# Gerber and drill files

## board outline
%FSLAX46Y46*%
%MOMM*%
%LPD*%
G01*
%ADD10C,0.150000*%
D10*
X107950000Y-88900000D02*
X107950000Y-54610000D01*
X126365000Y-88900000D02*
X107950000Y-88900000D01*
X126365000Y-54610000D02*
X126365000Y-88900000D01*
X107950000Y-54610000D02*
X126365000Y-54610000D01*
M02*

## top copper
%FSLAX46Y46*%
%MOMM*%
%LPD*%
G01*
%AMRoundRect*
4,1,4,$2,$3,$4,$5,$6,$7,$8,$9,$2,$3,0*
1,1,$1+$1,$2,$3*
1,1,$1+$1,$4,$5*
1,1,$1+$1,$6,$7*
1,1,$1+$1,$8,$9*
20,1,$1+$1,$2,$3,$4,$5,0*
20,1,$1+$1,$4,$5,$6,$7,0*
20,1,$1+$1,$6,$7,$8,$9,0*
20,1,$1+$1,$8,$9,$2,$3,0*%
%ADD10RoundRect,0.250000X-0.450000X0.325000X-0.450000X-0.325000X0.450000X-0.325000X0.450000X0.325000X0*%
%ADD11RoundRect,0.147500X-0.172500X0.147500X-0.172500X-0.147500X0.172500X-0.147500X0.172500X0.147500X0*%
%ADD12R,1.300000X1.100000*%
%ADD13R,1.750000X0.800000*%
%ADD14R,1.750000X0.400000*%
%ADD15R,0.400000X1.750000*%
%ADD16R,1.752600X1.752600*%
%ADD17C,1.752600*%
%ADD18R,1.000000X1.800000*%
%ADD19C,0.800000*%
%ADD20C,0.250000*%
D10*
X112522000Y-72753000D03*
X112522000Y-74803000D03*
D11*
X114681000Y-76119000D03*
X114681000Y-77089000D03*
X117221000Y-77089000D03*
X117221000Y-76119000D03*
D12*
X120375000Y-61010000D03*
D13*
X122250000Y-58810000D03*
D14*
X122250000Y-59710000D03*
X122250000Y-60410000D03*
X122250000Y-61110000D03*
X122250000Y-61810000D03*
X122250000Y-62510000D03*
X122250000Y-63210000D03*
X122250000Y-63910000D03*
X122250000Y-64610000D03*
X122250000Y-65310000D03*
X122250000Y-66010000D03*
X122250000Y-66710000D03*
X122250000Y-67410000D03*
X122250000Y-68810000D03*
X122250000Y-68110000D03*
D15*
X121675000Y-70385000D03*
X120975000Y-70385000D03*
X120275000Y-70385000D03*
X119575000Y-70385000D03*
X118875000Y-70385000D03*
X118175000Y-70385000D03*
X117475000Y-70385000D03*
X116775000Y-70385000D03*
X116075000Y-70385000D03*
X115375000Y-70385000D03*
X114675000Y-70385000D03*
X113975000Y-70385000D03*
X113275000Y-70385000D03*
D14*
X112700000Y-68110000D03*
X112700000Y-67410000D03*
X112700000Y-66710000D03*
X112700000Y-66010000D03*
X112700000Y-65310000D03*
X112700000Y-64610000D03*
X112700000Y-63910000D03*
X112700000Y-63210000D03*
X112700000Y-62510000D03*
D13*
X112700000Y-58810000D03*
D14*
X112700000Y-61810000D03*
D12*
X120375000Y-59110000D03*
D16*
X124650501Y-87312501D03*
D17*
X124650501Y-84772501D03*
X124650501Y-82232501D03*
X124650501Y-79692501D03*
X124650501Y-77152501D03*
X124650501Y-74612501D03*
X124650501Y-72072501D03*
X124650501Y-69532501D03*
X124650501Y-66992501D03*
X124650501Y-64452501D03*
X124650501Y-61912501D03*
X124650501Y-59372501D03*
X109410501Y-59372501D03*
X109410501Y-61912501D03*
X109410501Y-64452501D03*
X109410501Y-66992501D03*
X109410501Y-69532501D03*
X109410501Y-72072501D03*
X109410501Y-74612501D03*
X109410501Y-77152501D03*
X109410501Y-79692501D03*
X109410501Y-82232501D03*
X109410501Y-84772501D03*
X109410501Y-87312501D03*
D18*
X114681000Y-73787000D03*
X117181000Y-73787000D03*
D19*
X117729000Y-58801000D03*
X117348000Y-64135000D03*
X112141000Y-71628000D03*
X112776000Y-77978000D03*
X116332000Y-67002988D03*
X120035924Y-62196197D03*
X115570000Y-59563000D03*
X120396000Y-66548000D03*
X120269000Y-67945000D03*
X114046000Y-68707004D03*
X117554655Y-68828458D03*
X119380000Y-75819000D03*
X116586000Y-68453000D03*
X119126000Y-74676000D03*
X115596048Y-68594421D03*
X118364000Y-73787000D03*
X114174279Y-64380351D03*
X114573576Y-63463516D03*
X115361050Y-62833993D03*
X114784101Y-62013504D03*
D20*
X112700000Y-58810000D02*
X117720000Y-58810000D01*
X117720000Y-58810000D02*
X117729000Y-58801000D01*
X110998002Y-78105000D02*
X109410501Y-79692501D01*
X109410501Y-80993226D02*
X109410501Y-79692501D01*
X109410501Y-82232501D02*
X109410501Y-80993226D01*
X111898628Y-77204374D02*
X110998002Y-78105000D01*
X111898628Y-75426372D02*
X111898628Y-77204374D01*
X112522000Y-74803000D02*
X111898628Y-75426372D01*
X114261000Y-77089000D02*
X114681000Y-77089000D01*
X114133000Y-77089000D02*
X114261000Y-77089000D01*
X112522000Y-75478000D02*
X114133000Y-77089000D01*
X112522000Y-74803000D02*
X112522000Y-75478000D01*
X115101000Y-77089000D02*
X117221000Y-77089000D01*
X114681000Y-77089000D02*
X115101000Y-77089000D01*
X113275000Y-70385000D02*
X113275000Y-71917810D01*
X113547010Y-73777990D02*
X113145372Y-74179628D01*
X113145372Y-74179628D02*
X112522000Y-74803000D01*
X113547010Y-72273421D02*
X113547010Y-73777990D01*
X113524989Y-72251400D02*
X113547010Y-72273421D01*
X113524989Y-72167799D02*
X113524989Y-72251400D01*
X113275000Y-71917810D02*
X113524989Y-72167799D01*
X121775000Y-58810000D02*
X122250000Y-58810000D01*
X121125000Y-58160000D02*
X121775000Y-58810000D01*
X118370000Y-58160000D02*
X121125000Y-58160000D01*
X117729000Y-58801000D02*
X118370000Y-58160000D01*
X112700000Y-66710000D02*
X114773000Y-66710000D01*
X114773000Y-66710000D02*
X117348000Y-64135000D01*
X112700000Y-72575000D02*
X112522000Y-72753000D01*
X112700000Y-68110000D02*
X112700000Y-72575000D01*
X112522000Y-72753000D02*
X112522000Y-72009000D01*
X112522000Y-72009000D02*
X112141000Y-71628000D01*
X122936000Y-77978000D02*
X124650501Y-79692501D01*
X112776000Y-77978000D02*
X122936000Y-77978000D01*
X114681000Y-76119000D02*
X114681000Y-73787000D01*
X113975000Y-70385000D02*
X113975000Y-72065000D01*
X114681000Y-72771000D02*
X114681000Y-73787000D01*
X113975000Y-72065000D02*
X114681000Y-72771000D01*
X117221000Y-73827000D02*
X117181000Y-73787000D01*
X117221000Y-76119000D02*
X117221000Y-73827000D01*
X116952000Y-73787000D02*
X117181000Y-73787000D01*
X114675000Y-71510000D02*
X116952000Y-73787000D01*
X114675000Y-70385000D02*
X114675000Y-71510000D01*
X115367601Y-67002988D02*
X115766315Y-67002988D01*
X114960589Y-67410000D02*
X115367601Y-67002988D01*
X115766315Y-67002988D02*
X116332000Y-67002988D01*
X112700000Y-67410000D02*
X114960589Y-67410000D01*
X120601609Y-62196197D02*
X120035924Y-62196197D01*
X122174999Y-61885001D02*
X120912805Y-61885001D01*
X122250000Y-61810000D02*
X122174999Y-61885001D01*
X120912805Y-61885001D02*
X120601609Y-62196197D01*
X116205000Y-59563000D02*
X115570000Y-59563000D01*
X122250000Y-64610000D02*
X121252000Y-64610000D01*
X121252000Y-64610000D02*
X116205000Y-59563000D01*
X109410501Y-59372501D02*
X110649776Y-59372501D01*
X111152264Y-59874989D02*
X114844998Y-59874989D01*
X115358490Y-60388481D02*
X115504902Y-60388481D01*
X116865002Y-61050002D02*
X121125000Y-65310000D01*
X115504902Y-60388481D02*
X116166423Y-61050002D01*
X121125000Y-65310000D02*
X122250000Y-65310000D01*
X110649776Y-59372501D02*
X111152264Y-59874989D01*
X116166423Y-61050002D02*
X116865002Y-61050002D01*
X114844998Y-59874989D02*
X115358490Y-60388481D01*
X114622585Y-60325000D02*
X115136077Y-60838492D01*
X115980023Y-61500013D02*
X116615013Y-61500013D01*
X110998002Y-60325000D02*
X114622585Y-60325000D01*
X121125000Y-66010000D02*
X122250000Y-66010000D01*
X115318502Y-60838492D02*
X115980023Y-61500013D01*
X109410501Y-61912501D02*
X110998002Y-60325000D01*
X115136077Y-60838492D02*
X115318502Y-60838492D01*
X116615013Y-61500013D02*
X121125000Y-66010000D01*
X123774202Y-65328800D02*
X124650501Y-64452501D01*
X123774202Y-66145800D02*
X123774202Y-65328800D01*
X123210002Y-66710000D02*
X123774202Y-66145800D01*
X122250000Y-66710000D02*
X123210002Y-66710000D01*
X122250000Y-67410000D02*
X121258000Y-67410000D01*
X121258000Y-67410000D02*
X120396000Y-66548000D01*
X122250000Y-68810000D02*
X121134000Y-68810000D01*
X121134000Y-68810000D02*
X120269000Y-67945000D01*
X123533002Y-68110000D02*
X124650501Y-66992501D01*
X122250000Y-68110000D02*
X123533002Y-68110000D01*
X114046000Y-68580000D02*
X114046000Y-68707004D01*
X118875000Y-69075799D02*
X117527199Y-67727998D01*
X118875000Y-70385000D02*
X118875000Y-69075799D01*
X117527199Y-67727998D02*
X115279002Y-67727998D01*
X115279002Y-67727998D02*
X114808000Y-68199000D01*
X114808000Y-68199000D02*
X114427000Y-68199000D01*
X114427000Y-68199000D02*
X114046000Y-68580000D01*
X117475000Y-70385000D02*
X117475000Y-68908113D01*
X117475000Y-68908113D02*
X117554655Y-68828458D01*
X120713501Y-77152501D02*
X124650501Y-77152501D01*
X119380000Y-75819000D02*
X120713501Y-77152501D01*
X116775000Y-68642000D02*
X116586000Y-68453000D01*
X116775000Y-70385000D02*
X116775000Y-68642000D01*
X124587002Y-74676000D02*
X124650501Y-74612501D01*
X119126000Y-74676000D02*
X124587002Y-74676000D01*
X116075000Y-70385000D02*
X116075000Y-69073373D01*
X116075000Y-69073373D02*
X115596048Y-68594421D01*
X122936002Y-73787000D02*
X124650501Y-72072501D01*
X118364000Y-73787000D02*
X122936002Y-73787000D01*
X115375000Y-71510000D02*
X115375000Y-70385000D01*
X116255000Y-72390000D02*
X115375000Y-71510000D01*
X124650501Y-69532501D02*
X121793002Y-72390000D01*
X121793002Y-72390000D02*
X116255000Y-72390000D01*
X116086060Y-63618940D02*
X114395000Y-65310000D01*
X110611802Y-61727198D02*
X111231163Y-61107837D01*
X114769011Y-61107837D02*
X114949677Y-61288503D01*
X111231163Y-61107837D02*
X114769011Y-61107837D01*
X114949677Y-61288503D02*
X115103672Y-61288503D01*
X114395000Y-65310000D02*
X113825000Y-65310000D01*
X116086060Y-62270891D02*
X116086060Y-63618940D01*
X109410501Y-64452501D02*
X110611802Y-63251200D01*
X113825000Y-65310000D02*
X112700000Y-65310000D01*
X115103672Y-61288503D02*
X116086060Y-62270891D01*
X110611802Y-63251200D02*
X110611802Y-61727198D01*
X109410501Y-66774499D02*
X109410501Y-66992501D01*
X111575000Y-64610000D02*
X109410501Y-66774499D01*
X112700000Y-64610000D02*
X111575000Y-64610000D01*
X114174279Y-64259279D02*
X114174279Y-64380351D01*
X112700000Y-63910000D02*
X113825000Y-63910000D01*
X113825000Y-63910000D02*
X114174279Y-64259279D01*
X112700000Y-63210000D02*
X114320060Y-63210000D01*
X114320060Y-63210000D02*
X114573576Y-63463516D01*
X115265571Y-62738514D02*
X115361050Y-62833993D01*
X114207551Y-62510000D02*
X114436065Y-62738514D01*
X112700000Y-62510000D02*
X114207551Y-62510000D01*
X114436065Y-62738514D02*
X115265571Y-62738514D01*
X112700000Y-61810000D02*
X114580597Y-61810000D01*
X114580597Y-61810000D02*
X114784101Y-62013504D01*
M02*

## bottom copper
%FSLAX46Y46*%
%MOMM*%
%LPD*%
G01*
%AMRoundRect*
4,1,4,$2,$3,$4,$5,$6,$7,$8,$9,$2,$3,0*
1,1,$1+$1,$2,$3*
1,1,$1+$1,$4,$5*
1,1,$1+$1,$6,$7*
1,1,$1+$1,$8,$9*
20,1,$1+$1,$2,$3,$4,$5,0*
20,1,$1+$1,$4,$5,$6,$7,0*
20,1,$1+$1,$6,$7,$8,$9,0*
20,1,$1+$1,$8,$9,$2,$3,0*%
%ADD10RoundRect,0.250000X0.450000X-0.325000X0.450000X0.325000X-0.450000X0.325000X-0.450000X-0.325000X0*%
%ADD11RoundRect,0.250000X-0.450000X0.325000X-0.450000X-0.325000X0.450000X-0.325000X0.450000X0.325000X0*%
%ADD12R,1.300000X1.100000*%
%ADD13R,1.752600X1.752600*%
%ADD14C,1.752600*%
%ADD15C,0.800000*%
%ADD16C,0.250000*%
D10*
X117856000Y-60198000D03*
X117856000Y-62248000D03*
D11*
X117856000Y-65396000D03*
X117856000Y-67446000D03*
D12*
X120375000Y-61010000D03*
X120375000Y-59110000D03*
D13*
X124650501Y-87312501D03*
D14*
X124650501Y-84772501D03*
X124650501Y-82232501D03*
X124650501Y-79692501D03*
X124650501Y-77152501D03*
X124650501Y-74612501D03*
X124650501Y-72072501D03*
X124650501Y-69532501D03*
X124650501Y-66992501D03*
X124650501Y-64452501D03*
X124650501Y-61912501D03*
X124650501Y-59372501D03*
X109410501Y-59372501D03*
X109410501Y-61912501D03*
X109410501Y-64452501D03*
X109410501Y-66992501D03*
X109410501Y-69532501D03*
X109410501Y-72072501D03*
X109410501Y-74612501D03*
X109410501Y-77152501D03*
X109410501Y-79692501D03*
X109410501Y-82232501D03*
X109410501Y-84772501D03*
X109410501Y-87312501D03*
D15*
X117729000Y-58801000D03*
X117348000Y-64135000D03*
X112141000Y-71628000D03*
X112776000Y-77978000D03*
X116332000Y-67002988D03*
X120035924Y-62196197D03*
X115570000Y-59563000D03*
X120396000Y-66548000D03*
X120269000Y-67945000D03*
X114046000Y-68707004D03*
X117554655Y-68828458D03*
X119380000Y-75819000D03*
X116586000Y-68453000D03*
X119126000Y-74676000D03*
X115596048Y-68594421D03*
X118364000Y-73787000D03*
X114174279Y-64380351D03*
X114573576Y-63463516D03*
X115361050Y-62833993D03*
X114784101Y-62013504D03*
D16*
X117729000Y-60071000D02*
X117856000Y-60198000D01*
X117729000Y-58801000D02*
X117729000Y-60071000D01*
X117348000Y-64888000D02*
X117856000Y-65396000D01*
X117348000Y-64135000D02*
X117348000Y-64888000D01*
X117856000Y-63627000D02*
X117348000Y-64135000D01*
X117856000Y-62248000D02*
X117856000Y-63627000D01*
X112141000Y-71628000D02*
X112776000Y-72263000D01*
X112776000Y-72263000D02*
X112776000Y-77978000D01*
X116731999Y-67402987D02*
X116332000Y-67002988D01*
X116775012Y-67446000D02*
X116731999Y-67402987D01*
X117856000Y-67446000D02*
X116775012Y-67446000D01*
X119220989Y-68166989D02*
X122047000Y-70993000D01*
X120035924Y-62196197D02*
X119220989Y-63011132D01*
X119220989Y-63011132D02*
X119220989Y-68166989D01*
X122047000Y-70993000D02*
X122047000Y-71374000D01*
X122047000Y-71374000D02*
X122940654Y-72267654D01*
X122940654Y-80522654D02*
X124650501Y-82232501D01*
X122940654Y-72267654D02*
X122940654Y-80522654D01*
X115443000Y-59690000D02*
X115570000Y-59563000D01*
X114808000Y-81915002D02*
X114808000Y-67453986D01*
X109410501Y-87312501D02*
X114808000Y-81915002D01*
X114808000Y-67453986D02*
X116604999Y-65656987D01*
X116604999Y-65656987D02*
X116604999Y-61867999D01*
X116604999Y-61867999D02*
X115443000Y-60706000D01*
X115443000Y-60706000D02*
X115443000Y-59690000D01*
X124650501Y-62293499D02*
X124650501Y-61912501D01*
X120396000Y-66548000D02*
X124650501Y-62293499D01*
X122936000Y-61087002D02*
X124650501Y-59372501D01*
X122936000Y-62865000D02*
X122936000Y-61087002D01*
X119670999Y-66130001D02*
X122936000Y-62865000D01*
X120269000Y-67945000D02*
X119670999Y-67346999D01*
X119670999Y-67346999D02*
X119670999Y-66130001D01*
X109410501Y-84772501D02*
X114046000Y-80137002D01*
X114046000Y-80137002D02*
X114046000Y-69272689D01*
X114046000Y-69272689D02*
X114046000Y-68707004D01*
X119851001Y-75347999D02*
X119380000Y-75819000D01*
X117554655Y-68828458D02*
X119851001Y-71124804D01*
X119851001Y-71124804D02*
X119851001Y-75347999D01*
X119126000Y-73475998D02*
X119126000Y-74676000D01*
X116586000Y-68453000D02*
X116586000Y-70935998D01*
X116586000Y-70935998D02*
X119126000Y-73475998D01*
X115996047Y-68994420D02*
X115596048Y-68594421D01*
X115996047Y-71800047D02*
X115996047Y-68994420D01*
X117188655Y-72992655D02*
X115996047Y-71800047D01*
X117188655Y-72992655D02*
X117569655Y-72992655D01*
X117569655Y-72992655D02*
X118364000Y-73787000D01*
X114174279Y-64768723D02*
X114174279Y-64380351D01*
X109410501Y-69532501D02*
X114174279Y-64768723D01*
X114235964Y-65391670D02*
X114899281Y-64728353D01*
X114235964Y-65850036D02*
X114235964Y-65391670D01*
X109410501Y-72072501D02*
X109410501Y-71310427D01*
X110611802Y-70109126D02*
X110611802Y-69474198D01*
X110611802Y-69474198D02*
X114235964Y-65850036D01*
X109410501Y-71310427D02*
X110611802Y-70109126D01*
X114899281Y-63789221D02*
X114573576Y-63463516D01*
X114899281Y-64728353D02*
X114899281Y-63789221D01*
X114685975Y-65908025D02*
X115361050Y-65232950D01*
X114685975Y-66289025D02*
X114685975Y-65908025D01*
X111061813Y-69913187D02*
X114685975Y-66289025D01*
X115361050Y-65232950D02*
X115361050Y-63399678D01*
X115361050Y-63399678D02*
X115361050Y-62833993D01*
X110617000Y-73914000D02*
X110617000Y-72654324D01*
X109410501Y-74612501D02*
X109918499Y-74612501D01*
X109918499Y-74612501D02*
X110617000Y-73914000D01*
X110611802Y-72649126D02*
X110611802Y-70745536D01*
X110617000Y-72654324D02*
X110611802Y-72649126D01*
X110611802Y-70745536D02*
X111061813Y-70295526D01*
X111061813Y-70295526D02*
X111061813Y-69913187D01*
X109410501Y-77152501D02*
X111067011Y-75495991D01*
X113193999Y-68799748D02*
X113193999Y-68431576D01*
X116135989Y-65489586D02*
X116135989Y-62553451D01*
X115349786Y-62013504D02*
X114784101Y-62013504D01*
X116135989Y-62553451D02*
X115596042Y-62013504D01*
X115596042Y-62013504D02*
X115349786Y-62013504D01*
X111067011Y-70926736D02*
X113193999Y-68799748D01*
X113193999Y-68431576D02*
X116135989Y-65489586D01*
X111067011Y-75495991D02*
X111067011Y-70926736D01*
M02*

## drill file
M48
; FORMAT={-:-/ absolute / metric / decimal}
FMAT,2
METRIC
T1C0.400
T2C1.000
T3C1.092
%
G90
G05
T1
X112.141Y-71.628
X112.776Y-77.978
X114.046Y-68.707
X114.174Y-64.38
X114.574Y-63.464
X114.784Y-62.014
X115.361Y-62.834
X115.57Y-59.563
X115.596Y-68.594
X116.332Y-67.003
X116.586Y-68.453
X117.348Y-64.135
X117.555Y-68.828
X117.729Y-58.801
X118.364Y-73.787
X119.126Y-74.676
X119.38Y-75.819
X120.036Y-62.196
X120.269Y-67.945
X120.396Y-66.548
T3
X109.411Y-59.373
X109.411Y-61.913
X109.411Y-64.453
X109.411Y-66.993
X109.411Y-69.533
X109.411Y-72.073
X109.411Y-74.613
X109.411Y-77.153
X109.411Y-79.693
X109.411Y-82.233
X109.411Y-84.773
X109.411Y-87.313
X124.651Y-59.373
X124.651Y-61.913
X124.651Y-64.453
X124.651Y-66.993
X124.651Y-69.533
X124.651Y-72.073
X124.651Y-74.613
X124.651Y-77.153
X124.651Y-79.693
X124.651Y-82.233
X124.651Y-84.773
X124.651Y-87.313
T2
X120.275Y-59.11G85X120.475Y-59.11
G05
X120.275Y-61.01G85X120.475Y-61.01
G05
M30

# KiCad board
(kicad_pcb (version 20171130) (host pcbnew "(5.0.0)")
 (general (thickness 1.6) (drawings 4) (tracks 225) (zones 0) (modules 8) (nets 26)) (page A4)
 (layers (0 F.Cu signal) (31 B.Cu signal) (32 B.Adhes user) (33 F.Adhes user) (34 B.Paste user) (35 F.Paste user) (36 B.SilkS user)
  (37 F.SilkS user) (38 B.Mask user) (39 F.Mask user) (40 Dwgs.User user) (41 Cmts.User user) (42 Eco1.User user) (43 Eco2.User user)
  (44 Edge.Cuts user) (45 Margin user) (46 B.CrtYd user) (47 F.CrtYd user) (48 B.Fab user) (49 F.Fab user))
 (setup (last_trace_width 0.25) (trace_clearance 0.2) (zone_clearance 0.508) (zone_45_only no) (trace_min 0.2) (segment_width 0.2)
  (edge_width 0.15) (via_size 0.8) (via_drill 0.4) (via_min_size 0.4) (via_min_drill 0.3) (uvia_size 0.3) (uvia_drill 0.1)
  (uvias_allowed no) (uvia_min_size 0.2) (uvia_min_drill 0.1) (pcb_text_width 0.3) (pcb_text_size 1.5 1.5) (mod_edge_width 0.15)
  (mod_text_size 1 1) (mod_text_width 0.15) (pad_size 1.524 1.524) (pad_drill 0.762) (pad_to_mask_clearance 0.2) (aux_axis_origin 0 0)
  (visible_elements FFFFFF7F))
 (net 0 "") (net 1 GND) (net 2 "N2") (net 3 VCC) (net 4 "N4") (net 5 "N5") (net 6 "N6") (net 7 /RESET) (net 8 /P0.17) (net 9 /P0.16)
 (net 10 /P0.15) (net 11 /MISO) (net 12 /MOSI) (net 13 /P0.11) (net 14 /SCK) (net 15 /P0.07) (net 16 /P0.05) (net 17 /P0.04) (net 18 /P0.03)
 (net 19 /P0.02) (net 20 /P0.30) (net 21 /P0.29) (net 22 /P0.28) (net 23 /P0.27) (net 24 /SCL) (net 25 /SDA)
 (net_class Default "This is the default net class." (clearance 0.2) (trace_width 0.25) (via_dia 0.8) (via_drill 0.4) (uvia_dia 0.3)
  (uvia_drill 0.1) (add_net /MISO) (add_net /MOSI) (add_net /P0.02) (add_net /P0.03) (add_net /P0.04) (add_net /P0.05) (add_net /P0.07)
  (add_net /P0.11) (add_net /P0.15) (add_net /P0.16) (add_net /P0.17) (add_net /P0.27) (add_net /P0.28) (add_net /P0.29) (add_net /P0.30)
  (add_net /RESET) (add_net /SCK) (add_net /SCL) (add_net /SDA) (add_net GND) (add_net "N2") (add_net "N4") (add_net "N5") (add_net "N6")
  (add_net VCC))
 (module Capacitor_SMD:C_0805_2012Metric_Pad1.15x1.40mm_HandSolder (layer B.Cu) (at 117.856 61.223 90)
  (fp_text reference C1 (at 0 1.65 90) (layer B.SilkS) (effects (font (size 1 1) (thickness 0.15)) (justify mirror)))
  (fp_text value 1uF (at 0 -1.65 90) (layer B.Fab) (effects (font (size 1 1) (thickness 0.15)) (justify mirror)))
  (pad 2 smd roundrect (at 1.025 0 90) (size 1.15 1.4) (layers B.Cu B.Paste B.Mask) (roundrect_rratio 0.217391) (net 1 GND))
  (pad 1 smd roundrect (at -1.025 0 90) (size 1.15 1.4) (layers B.Cu B.Paste B.Mask) (roundrect_rratio 0.217391) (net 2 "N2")))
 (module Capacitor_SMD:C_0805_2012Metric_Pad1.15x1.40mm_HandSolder (layer F.Cu) (at 112.522 73.778 270)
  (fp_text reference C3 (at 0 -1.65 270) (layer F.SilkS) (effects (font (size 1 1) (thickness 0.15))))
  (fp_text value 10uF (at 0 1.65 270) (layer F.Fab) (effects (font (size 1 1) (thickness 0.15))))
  (pad 1 smd roundrect (at -1.025 0 270) (size 1.15 1.4) (layers F.Cu F.Paste F.Mask) (roundrect_rratio 0.217391) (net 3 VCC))
  (pad 2 smd roundrect (at 1.025 0 270) (size 1.15 1.4) (layers F.Cu F.Paste F.Mask) (roundrect_rratio 0.217391) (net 1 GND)))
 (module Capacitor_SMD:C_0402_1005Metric (layer F.Cu) (at 114.681 76.604 270)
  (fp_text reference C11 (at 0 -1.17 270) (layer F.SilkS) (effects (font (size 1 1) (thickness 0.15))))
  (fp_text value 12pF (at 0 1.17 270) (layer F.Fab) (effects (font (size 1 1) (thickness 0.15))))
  (pad 1 smd roundrect (at -0.485 0 270) (size 0.59 0.64) (layers F.Cu F.Paste F.Mask) (roundrect_rratio 0.25) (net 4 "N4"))
  (pad 2 smd roundrect (at 0.485 0 270) (size 0.59 0.64) (layers F.Cu F.Paste F.Mask) (roundrect_rratio 0.25) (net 1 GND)))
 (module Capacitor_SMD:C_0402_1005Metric (layer F.Cu) (at 117.221 76.604 270)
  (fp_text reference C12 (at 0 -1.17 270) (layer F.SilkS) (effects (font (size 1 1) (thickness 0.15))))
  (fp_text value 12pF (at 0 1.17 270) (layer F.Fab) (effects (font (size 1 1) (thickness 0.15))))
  (pad 2 smd roundrect (at 0.485 0 270) (size 0.59 0.64) (layers F.Cu F.Paste F.Mask) (roundrect_rratio 0.25) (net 1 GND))
  (pad 1 smd roundrect (at -0.485 0 270) (size 0.59 0.64) (layers F.Cu F.Paste F.Mask) (roundrect_rratio 0.25) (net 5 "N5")))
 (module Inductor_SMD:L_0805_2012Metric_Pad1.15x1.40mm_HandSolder (layer B.Cu) (at 117.856 66.421 270)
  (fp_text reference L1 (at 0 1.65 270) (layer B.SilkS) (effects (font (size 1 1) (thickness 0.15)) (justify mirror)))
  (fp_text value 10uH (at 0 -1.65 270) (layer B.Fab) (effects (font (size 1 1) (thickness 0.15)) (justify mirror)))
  (pad 1 smd roundrect (at -1.025 0 270) (size 1.15 1.4) (layers B.Cu B.Paste B.Mask) (roundrect_rratio 0.217391) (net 2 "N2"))
  (pad 2 smd roundrect (at 1.025 0 270) (size 1.15 1.4) (layers B.Cu B.Paste B.Mask) (roundrect_rratio 0.217391) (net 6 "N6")))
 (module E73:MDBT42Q (layer F.Cu) (at 117.475 54.61)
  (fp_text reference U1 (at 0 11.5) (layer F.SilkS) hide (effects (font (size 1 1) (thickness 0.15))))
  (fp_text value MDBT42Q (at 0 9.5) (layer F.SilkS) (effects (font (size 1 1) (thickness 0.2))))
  (pad 41 thru_hole rect (at 2.9 6.4) (size 1.3 1.1) (drill oval 1.2 1) (layers *.Cu *.Mask))
  (pad 39 smd rect (at 4.775 4.2) (size 1.75 0.8) (layers F.Cu F.Paste F.Mask) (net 1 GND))
  (pad 38 smd rect (at 4.775 5.1) (size 1.75 0.4) (layers F.Cu F.Paste F.Mask))
  (pad 37 smd rect (at 4.775 5.8) (size 1.75 0.4) (layers F.Cu F.Paste F.Mask))
  (pad 36 smd rect (at 4.775 6.5) (size 1.75 0.4) (layers F.Cu F.Paste F.Mask))
  (pad 35 smd rect (at 4.775 7.2) (size 1.75 0.4) (layers F.Cu F.Paste F.Mask) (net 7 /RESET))
  (pad 34 smd rect (at 4.775 7.9) (size 1.75 0.4) (layers F.Cu F.Paste F.Mask))
  (pad 33 smd rect (at 4.775 8.6) (size 1.75 0.4) (layers F.Cu F.Paste F.Mask))
  (pad 32 smd rect (at 4.775 9.3) (size 1.75 0.4) (layers F.Cu F.Paste F.Mask))
  (pad 31 smd rect (at 4.775 10) (size 1.75 0.4) (layers F.Cu F.Paste F.Mask) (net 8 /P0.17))
  (pad 30 smd rect (at 4.775 10.7) (size 1.75 0.4) (layers F.Cu F.Paste F.Mask) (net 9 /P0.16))
  (pad 29 smd rect (at 4.775 11.4) (size 1.75 0.4) (layers F.Cu F.Paste F.Mask) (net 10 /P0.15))
  (pad 28 smd rect (at 4.775 12.1) (size 1.75 0.4) (layers F.Cu F.Paste F.Mask) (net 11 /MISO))
  (pad 27 smd rect (at 4.775 12.8) (size 1.75 0.4) (layers F.Cu F.Paste F.Mask) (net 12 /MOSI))
  (pad 25 smd rect (at 4.775 14.2) (size 1.75 0.4) (layers F.Cu F.Paste F.Mask) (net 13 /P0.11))
  (pad 26 smd rect (at 4.775 13.5) (size 1.75 0.4) (layers F.Cu F.Paste F.Mask) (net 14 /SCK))
  (pad 24 smd rect (at 4.2 15.775) (size 0.4 1.75) (layers F.Cu F.Paste F.Mask) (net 1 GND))
  (pad 23 smd rect (at 3.5 15.775) (size 0.4 1.75) (layers F.Cu F.Paste F.Mask))
  (pad 22 smd rect (at 2.8 15.775) (size 0.4 1.75) (layers F.Cu F.Paste F.Mask))
  (pad 21 smd rect (at 2.1 15.775) (size 0.4 1.75) (layers F.Cu F.Paste F.Mask))
  (pad 20 smd rect (at 1.4 15.775) (size 0.4 1.75) (layers F.Cu F.Paste F.Mask) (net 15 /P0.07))
  (pad 19 smd rect (at 0.7 15.775) (size 0.4 1.75) (layers F.Cu F.Paste F.Mask))
  (pad 18 smd rect (at 0 15.775) (size 0.4 1.75) (layers F.Cu F.Paste F.Mask) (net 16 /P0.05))
  (pad 17 smd rect (at -0.7 15.775) (size 0.4 1.75) (layers F.Cu F.Paste F.Mask) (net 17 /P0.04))
  (pad 16 smd rect (at -1.4 15.775) (size 0.4 1.75) (layers F.Cu F.Paste F.Mask) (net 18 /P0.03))
  (pad 15 smd rect (at -2.1 15.775) (size 0.4 1.75) (layers F.Cu F.Paste F.Mask) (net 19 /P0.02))
  (pad 14 smd rect (at -2.8 15.775) (size 0.4 1.75) (layers F.Cu F.Paste F.Mask) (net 5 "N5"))
  (pad 13 smd rect (at -3.5 15.775) (size 0.4 1.75) (layers F.Cu F.Paste F.Mask) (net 4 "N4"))
  (pad 12 smd rect (at -4.2 15.775) (size 0.4 1.75) (layers F.Cu F.Paste F.Mask) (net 1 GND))
  (pad 11 smd rect (at -4.775 13.5) (size 1.75 0.4) (layers F.Cu F.Paste F.Mask) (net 3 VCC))
  (pad 10 smd rect (at -4.775 12.8) (size 1.75 0.4) (layers F.Cu F.Paste F.Mask) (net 6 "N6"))
  (pad 9 smd rect (at -4.775 12.1) (size 1.75 0.4) (layers F.Cu F.Paste F.Mask) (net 2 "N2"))
  (pad 8 smd rect (at -4.775 11.4) (size 1.75 0.4) (layers F.Cu F.Paste F.Mask))
  (pad 7 smd rect (at -4.775 10.7) (size 1.75 0.4) (layers F.Cu F.Paste F.Mask) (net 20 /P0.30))
  (pad 6 smd rect (at -4.775 10) (size 1.75 0.4) (layers F.Cu F.Paste F.Mask) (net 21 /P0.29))
  (pad 5 smd rect (at -4.775 9.3) (size 1.75 0.4) (layers F.Cu F.Paste F.Mask) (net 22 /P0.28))
  (pad 4 smd rect (at -4.775 8.6) (size 1.75 0.4) (layers F.Cu F.Paste F.Mask) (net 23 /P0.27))
  (pad 3 smd rect (at -4.775 7.9) (size 1.75 0.4) (layers F.Cu F.Paste F.Mask) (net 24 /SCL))
  (pad 1 smd rect (at -4.775 4.2) (size 1.75 0.8) (layers F.Cu F.Paste F.Mask) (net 1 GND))
  (pad 2 smd rect (at -4.775 7.2) (size 1.75 0.4) (layers F.Cu F.Paste F.Mask) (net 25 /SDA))
  (pad 40 thru_hole rect (at 2.9 4.5) (size 1.3 1.1) (drill oval 1.2 1) (layers *.Cu *.Mask)))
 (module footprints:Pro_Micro (layer F.Cu) (at 117.030501 74.866501 180)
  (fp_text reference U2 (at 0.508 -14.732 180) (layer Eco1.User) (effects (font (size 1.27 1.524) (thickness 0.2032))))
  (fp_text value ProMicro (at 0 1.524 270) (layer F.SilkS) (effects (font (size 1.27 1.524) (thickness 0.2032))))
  (pad 1 thru_hole rect (at -7.62 -12.446 90) (size 1.7526 1.7526) (drill 1.0922) (layers *.Cu *.SilkS *.Mask))
  (pad 2 thru_hole circle (at -7.62 -9.906 90) (size 1.7526 1.7526) (drill 1.0922) (layers *.Cu *.SilkS *.Mask) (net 1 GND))
  (pad 3 thru_hole circle (at -7.62 -7.366 90) (size 1.7526 1.7526) (drill 1.0922) (layers *.Cu *.SilkS *.Mask) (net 7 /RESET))
  (pad 4 thru_hole circle (at -7.62 -4.826 90) (size 1.7526 1.7526) (drill 1.0922) (layers *.Cu *.SilkS *.Mask) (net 3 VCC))
  (pad 5 thru_hole circle (at -7.62 -2.286 90) (size 1.7526 1.7526) (drill 1.0922) (layers *.Cu *.SilkS *.Mask) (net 16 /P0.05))
  (pad 6 thru_hole circle (at -7.62 0.254 90) (size 1.7526 1.7526) (drill 1.0922) (layers *.Cu *.SilkS *.Mask) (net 17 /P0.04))
  (pad 7 thru_hole circle (at -7.62 2.794 90) (size 1.7526 1.7526) (drill 1.0922) (layers *.Cu *.SilkS *.Mask) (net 18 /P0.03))
  (pad 8 thru_hole circle (at -7.62 5.334 90) (size 1.7526 1.7526) (drill 1.0922) (layers *.Cu *.SilkS *.Mask) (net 19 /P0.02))
  (pad 9 thru_hole circle (at -7.62 7.874 90) (size 1.7526 1.7526) (drill 1.0922) (layers *.Cu *.SilkS *.Mask) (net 14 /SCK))
  (pad 10 thru_hole circle (at -7.62 10.414 90) (size 1.7526 1.7526) (drill 1.0922) (layers *.Cu *.SilkS *.Mask) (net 11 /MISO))
  (pad 11 thru_hole circle (at -7.62 12.954 90) (size 1.7526 1.7526) (drill 1.0922) (layers *.Cu *.SilkS *.Mask) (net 12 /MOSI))
  (pad 12 thru_hole circle (at -7.62 15.494 90) (size 1.7526 1.7526) (drill 1.0922) (layers *.Cu *.SilkS *.Mask) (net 13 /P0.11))
  (pad 24 thru_hole circle (at 7.62 15.494 90) (size 1.7526 1.7526) (drill 1.0922) (layers *.Cu *.SilkS *.Mask) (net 9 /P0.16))
  (pad 23 thru_hole circle (at 7.62 12.954 90) (size 1.7526 1.7526) (drill 1.0922) (layers *.Cu *.SilkS *.Mask) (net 10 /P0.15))
  (pad 22 thru_hole circle (at 7.62 10.414 90) (size 1.7526 1.7526) (drill 1.0922) (layers *.Cu *.SilkS *.Mask) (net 20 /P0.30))
  (pad 21 thru_hole circle (at 7.62 7.874 90) (size 1.7526 1.7526) (drill 1.0922) (layers *.Cu *.SilkS *.Mask) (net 21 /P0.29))
  (pad 20 thru_hole circle (at 7.62 5.334 90) (size 1.7526 1.7526) (drill 1.0922) (layers *.Cu *.SilkS *.Mask) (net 22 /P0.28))
  (pad 19 thru_hole circle (at 7.62 2.794 90) (size 1.7526 1.7526) (drill 1.0922) (layers *.Cu *.SilkS *.Mask) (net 23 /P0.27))
  (pad 18 thru_hole circle (at 7.62 0.254 90) (size 1.7526 1.7526) (drill 1.0922) (layers *.Cu *.SilkS *.Mask) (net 24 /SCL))
  (pad 17 thru_hole circle (at 7.62 -2.286 90) (size 1.7526 1.7526) (drill 1.0922) (layers *.Cu *.SilkS *.Mask) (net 25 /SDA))
  (pad 16 thru_hole circle (at 7.62 -4.826 90) (size 1.7526 1.7526) (drill 1.0922) (layers *.Cu *.SilkS *.Mask) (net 1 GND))
  (pad 15 thru_hole circle (at 7.62 -7.366 90) (size 1.7526 1.7526) (drill 1.0922) (layers *.Cu *.SilkS *.Mask) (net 1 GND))
  (pad 14 thru_hole circle (at 7.62 -9.906 90) (size 1.7526 1.7526) (drill 1.0922) (layers *.Cu *.SilkS *.Mask) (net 15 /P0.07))
  (pad 13 thru_hole circle (at 7.62 -12.446 90) (size 1.7526 1.7526) (drill 1.0922) (layers *.Cu *.SilkS *.Mask) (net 8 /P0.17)))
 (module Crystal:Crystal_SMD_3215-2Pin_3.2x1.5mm (layer F.Cu) (at 115.931 73.787 180)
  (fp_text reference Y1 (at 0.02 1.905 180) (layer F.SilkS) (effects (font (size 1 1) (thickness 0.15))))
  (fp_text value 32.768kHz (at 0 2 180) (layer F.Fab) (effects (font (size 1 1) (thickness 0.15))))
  (pad 1 smd rect (at 1.25 0 180) (size 1 1.8) (layers F.Cu F.Paste F.Mask) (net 4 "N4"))
  (pad 2 smd rect (at -1.25 0 180) (size 1 1.8) (layers F.Cu F.Paste F.Mask) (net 5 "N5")))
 (gr_line (start 107.95 88.9) (end 107.95 54.61) (layer Edge.Cuts) (width 0.15))
 (gr_line (start 126.365 88.9) (end 107.95 88.9) (layer Edge.Cuts) (width 0.15))
 (gr_line (start 126.365 54.61) (end 126.365 88.9) (layer Edge.Cuts) (width 0.15))
 (gr_line (start 107.95 54.61) (end 126.365 54.61) (layer Edge.Cuts) (width 0.15))
 (via (at 117.729 58.801) (size 0.8) (drill 0.4) (layers F.Cu B.Cu) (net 1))
 (segment (start 112.7 58.81) (end 117.72 58.81) (width 0.25) (layer F.Cu) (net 1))
 (segment (start 117.72 58.81) (end 117.729 58.801) (width 0.25) (layer F.Cu) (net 1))
 (segment (start 117.729 60.071) (end 117.856 60.198) (width 0.25) (layer B.Cu) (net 1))
 (segment (start 117.729 58.801) (end 117.729 60.071) (width 0.25) (layer B.Cu) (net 1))
 (segment (start 110.998002 78.105) (end 109.410501 79.692501) (width 0.25) (layer F.Cu) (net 1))
 (segment (start 109.410501 80.993226) (end 109.410501 79.692501) (width 0.25) (layer F.Cu) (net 1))
 (segment (start 109.410501 82.232501) (end 109.410501 80.993226) (width 0.25) (layer F.Cu) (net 1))
 (segment (start 111.898628 77.204374) (end 110.998002 78.105) (width 0.25) (layer F.Cu) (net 1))
 (segment (start 111.898628 75.426372) (end 111.898628 77.204374) (width 0.25) (layer F.Cu) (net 1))
 (segment (start 112.522 74.803) (end 111.898628 75.426372) (width 0.25) (layer F.Cu) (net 1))
 (segment (start 114.261 77.089) (end 114.681 77.089) (width 0.25) (layer F.Cu) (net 1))
 (segment (start 114.133 77.089) (end 114.261 77.089) (width 0.25) (layer F.Cu) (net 1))
 (segment (start 112.522 75.478) (end 114.133 77.089) (width 0.25) (layer F.Cu) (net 1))
 (segment (start 112.522 74.803) (end 112.522 75.478) (width 0.25) (layer F.Cu) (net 1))
 (segment (start 115.101 77.089) (end 117.221 77.089) (width 0.25) (layer F.Cu) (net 1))
 (segment (start 114.681 77.089) (end 115.101 77.089) (width 0.25) (layer F.Cu) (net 1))
 (segment (start 113.275 70.385) (end 113.275 71.91781) (width 0.25) (layer F.Cu) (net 1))
 (segment (start 113.54701 73.77799) (end 113.145372 74.179628) (width 0.25) (layer F.Cu) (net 1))
 (segment (start 113.145372 74.179628) (end 112.522 74.803) (width 0.25) (layer F.Cu) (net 1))
 (segment (start 113.54701 72.273421) (end 113.54701 73.77799) (width 0.25) (layer F.Cu) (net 1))
 (segment (start 113.524989 72.2514) (end 113.54701 72.273421) (width 0.25) (layer F.Cu) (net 1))
 (segment (start 113.524989 72.167799) (end 113.524989 72.2514) (width 0.25) (layer F.Cu) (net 1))
 (segment (start 113.275 71.91781) (end 113.524989 72.167799) (width 0.25) (layer F.Cu) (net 1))
 (segment (start 121.775 58.81) (end 122.25 58.81) (width 0.25) (layer F.Cu) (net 1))
 (segment (start 121.125 58.16) (end 121.775 58.81) (width 0.25) (layer F.Cu) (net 1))
 (segment (start 118.37 58.16) (end 121.125 58.16) (width 0.25) (layer F.Cu) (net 1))
 (segment (start 117.729 58.801) (end 118.37 58.16) (width 0.25) (layer F.Cu) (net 1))
 (via (at 117.348 64.135) (size 0.8) (drill 0.4) (layers F.Cu B.Cu) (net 2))
 (segment (start 112.7 66.71) (end 114.773 66.71) (width 0.25) (layer F.Cu) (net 2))
 (segment (start 114.773 66.71) (end 117.348 64.135) (width 0.25) (layer F.Cu) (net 2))
 (segment (start 117.348 64.888) (end 117.856 65.396) (width 0.25) (layer B.Cu) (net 2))
 (segment (start 117.348 64.135) (end 117.348 64.888) (width 0.25) (layer B.Cu) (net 2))
 (segment (start 117.856 63.627) (end 117.348 64.135) (width 0.25) (layer B.Cu) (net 2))
 (segment (start 117.856 62.248) (end 117.856 63.627) (width 0.25) (layer B.Cu) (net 2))
 (segment (start 112.7 72.575) (end 112.522 72.753) (width 0.25) (layer F.Cu) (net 3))
 (segment (start 112.7 68.11) (end 112.7 72.575) (width 0.25) (layer F.Cu) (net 3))
 (via (at 112.141 71.628) (size 0.8) (drill 0.4) (layers F.Cu B.Cu) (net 3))
 (segment (start 112.522 72.753) (end 112.522 72.009) (width 0.25) (layer F.Cu) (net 3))
 (segment (start 112.522 72.009) (end 112.141 71.628) (width 0.25) (layer F.Cu) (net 3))
 (via (at 112.776 77.978) (size 0.8) (drill 0.4) (layers F.Cu B.Cu) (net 3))
 (segment (start 112.141 71.628) (end 112.776 72.263) (width 0.25) (layer B.Cu) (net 3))
 (segment (start 112.776 72.263) (end 112.776 77.978) (width 0.25) (layer B.Cu) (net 3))
 (segment (start 122.936 77.978) (end 124.650501 79.692501) (width 0.25) (layer F.Cu) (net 3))
 (segment (start 112.776 77.978) (end 122.936 77.978) (width 0.25) (layer F.Cu) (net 3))
 (segment (start 114.681 76.119) (end 114.681 73.787) (width 0.25) (layer F.Cu) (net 4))
 (segment (start 113.975 70.385) (end 113.975 72.065) (width 0.25) (layer F.Cu) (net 4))
 (segment (start 114.681 72.771) (end 114.681 73.787) (width 0.25) (layer F.Cu) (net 4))
 (segment (start 113.975 72.065) (end 114.681 72.771) (width 0.25) (layer F.Cu) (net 4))
 (segment (start 117.221 73.827) (end 117.181 73.787) (width 0.25) (layer F.Cu) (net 5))
 (segment (start 117.221 76.119) (end 117.221 73.827) (width 0.25) (layer F.Cu) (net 5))
 (segment (start 116.952 73.787) (end 117.181 73.787) (width 0.25) (layer F.Cu) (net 5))
 (segment (start 114.675 71.51) (end 116.952 73.787) (width 0.25) (layer F.Cu) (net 5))
 (segment (start 114.675 70.385) (end 114.675 71.51) (width 0.25) (layer F.Cu) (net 5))
 (via (at 116.332 67.002988) (size 0.8) (drill 0.4) (layers F.Cu B.Cu) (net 6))
 (segment (start 116.731999 67.402987) (end 116.332 67.002988) (width 0.25) (layer B.Cu) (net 6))
 (segment (start 116.775012 67.446) (end 116.731999 67.402987) (width 0.25) (layer B.Cu) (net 6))
 (segment (start 117.856 67.446) (end 116.775012 67.446) (width 0.25) (layer B.Cu) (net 6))
 (segment (start 115.367601 67.002988) (end 115.766315 67.002988) (width 0.25) (layer F.Cu) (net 6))
 (segment (start 114.960589 67.41) (end 115.367601 67.002988) (width 0.25) (layer F.Cu) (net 6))
 (segment (start 115.766315 67.002988) (end 116.332 67.002988) (width 0.25) (layer F.Cu) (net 6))
 (segment (start 112.7 67.41) (end 114.960589 67.41) (width 0.25) (layer F.Cu) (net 6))
 (segment (start 120.601609 62.196197) (end 120.035924 62.196197) (width 0.25) (layer F.Cu) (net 7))
 (segment (start 122.174999 61.885001) (end 120.912805 61.885001) (width 0.25) (layer F.Cu) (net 7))
 (segment (start 122.25 61.81) (end 122.174999 61.885001) (width 0.25) (layer F.Cu) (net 7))
 (segment (start 120.912805 61.885001) (end 120.601609 62.196197) (width 0.25) (layer F.Cu) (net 7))
 (via (at 120.035924 62.196197) (size 0.8) (drill 0.4) (layers F.Cu B.Cu) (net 7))
 (segment (start 119.220989 68.166989) (end 122.047 70.993) (width 0.25) (layer B.Cu) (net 7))
 (segment (start 120.035924 62.196197) (end 119.220989 63.011132) (width 0.25) (layer B.Cu) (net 7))
 (segment (start 119.220989 63.011132) (end 119.220989 68.166989) (width 0.25) (layer B.Cu) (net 7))
 (segment (start 122.047 70.993) (end 122.047 71.374) (width 0.25) (layer B.Cu) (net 7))
 (segment (start 122.047 71.374) (end 122.940654 72.267654) (width 0.25) (layer B.Cu) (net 7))
 (segment (start 122.940654 80.522654) (end 124.650501 82.232501) (width 0.25) (layer B.Cu) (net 7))
 (segment (start 122.940654 72.267654) (end 122.940654 80.522654) (width 0.25) (layer B.Cu) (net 7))
 (via (at 115.57 59.563) (size 0.8) (drill 0.4) (layers F.Cu B.Cu) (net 8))
 (segment (start 115.443 59.69) (end 115.57 59.563) (width 0.25) (layer B.Cu) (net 8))
 (segment (start 114.808 81.915002) (end 114.808 67.453986) (width 0.25) (layer B.Cu) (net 8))
 (segment (start 109.410501 87.312501) (end 114.808 81.915002) (width 0.25) (layer B.Cu) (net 8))
 (segment (start 114.808 67.453986) (end 116.604999 65.656987) (width 0.25) (layer B.Cu) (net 8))
 (segment (start 116.604999 65.656987) (end 116.604999 61.867999) (width 0.25) (layer B.Cu) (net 8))
 (segment (start 116.604999 61.867999) (end 115.443 60.706) (width 0.25) (layer B.Cu) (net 8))
 (segment (start 115.443 60.706) (end 115.443 59.69) (width 0.25) (layer B.Cu) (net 8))
 (segment (start 116.205 59.563) (end 115.57 59.563) (width 0.25) (layer F.Cu) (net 8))
 (segment (start 122.25 64.61) (end 121.252 64.61) (width 0.25) (layer F.Cu) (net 8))
 (segment (start 121.252 64.61) (end 116.205 59.563) (width 0.25) (layer F.Cu) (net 8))
 (segment (start 109.410501 59.372501) (end 110.649776 59.372501) (width 0.25) (layer F.Cu) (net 9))
 (segment (start 111.152264 59.874989) (end 114.844998 59.874989) (width 0.25) (layer F.Cu) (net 9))
 (segment (start 115.35849 60.388481) (end 115.504902 60.388481) (width 0.25) (layer F.Cu) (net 9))
 (segment (start 116.865002 61.050002) (end 121.125 65.31) (width 0.25) (layer F.Cu) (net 9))
 (segment (start 115.504902 60.388481) (end 116.166423 61.050002) (width 0.25) (layer F.Cu) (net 9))
 (segment (start 121.125 65.31) (end 122.25 65.31) (width 0.25) (layer F.Cu) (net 9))
 (segment (start 110.649776 59.372501) (end 111.152264 59.874989) (width 0.25) (layer F.Cu) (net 9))
 (segment (start 116.166423 61.050002) (end 116.865002 61.050002) (width 0.25) (layer F.Cu) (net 9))
 (segment (start 114.844998 59.874989) (end 115.35849 60.388481) (width 0.25) (layer F.Cu) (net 9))
 (segment (start 114.622585 60.325) (end 115.136077 60.838492) (width 0.25) (layer F.Cu) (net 10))
 (segment (start 115.980023 61.500013) (end 116.615013 61.500013) (width 0.25) (layer F.Cu) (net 10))
 (segment (start 110.998002 60.325) (end 114.622585 60.325) (width 0.25) (layer F.Cu) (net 10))
 (segment (start 121.125 66.01) (end 122.25 66.01) (width 0.25) (layer F.Cu) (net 10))
 (segment (start 115.318502 60.838492) (end 115.980023 61.500013) (width 0.25) (layer F.Cu) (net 10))
 (segment (start 109.410501 61.912501) (end 110.998002 60.325) (width 0.25) (layer F.Cu) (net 10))
 (segment (start 115.136077 60.838492) (end 115.318502 60.838492) (width 0.25) (layer F.Cu) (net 10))
 (segment (start 116.615013 61.500013) (end 121.125 66.01) (width 0.25) (layer F.Cu) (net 10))
 (segment (start 123.774202 65.3288) (end 124.650501 64.452501) (width 0.25) (layer F.Cu) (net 11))
 (segment (start 123.774202 66.1458) (end 123.774202 65.3288) (width 0.25) (layer F.Cu) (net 11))
 (segment (start 123.210002 66.71) (end 123.774202 66.1458) (width 0.25) (layer F.Cu) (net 11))
 (segment (start 122.25 66.71) (end 123.210002 66.71) (width 0.25) (layer F.Cu) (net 11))
 (via (at 120.396 66.548) (size 0.8) (drill 0.4) (layers F.Cu B.Cu) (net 12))
 (segment (start 122.25 67.41) (end 121.258 67.41) (width 0.25) (layer F.Cu) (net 12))
 (segment (start 121.258 67.41) (end 120.396 66.548) (width 0.25) (layer F.Cu) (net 12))
 (segment (start 124.650501 62.293499) (end 124.650501 61.912501) (width 0.25) (layer B.Cu) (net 12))
 (segment (start 120.396 66.548) (end 124.650501 62.293499) (width 0.25) (layer B.Cu) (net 12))
 (via (at 120.269 67.945) (size 0.8) (drill 0.4) (layers F.Cu B.Cu) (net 13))
 (segment (start 122.25 68.81) (end 121.134 68.81) (width 0.25) (layer F.Cu) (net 13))
 (segment (start 121.134 68.81) (end 120.269 67.945) (width 0.25) (layer F.Cu) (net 13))
 (segment (start 122.936 61.087002) (end 124.650501 59.372501) (width 0.25) (layer B.Cu) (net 13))
 (segment (start 122.936 62.865) (end 122.936 61.087002) (width 0.25) (layer B.Cu) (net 13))
 (segment (start 119.670999 66.130001) (end 122.936 62.865) (width 0.25) (layer B.Cu) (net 13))
 (segment (start 120.269 67.945) (end 119.670999 67.346999) (width 0.25) (layer B.Cu) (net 13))
 (segment (start 119.670999 67.346999) (end 119.670999 66.130001) (width 0.25) (layer B.Cu) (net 13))
 (segment (start 123.533002 68.11) (end 124.650501 66.992501) (width 0.25) (layer F.Cu) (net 14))
 (segment (start 122.25 68.11) (end 123.533002 68.11) (width 0.25) (layer F.Cu) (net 14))
 (segment (start 109.410501 84.772501) (end 114.046 80.137002) (width 0.25) (layer B.Cu) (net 15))
 (via (at 114.046 68.707004) (size 0.8) (drill 0.4) (layers F.Cu B.Cu) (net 15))
 (segment (start 114.046 80.137002) (end 114.046 69.272689) (width 0.25) (layer B.Cu) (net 15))
 (segment (start 114.046 69.272689) (end 114.046 68.707004) (width 0.25) (layer B.Cu) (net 15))
 (segment (start 114.046 68.58) (end 114.046 68.707004) (width 0.25) (layer F.Cu) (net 15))
 (segment (start 118.875 69.075799) (end 117.527199 67.727998) (width 0.25) (layer F.Cu) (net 15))
 (segment (start 118.875 70.385) (end 118.875 69.075799) (width 0.25) (layer F.Cu) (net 15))
 (segment (start 117.527199 67.727998) (end 115.279002 67.727998) (width 0.25) (layer F.Cu) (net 15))
 (segment (start 115.279002 67.727998) (end 114.808 68.199) (width 0.25) (layer F.Cu) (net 15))
 (segment (start 114.808 68.199) (end 114.427 68.199) (width 0.25) (layer F.Cu) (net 15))
 (segment (start 114.427 68.199) (end 114.046 68.58) (width 0.25) (layer F.Cu) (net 15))
 (segment (start 117.475 70.385) (end 117.475 68.908113) (width 0.25) (layer F.Cu) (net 16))
 (segment (start 117.475 68.908113) (end 117.554655 68.828458) (width 0.25) (layer F.Cu) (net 16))
 (via (at 117.554655 68.828458) (size 0.8) (drill 0.4) (layers F.Cu B.Cu) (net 16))
 (via (at 119.38 75.819) (size 0.8) (drill 0.4) (layers F.Cu B.Cu) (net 16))
 (segment (start 119.851001 75.347999) (end 119.38 75.819) (width 0.25) (layer B.Cu) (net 16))
 (segment (start 117.554655 68.828458) (end 119.851001 71.124804) (width 0.25) (layer B.Cu) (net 16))
 (segment (start 119.851001 71.124804) (end 119.851001 75.347999) (width 0.25) (layer B.Cu) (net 16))
 (segment (start 120.713501 77.152501) (end 124.650501 77.152501) (width 0.25) (layer F.Cu) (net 16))
 (segment (start 119.38 75.819) (end 120.713501 77.152501) (width 0.25) (layer F.Cu) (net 16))
 (segment (start 116.775 68.642) (end 116.586 68.453) (width 0.25) (layer F.Cu) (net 17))
 (via (at 116.586 68.453) (size 0.8) (drill 0.4) (layers F.Cu B.Cu) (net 17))
 (segment (start 116.775 70.385) (end 116.775 68.642) (width 0.25) (layer F.Cu) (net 17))
 (via (at 119.126 74.676) (size 0.8) (drill 0.4) (layers F.Cu B.Cu) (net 17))
 (segment (start 119.126 73.475998) (end 119.126 74.676) (width 0.25) (layer B.Cu) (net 17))
 (segment (start 116.586 68.453) (end 116.586 70.935998) (width 0.25) (layer B.Cu) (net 17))
 (segment (start 116.586 70.935998) (end 119.126 73.475998) (width 0.25) (layer B.Cu) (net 17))
 (segment (start 124.587002 74.676) (end 124.650501 74.612501) (width 0.25) (layer F.Cu) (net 17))
 (segment (start 119.126 74.676) (end 124.587002 74.676) (width 0.25) (layer F.Cu) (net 17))
 (via (at 115.596048 68.594421) (size 0.8) (drill 0.4) (layers F.Cu B.Cu) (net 18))
 (segment (start 116.075 70.385) (end 116.075 69.073373) (width 0.25) (layer F.Cu) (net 18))
 (segment (start 116.075 69.073373) (end 115.596048 68.594421) (width 0.25) (layer F.Cu) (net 18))
 (segment (start 115.996047 68.99442) (end 115.596048 68.594421) (width 0.25) (layer B.Cu) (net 18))
 (segment (start 115.996047 71.800047) (end 115.996047 68.99442) (width 0.25) (layer B.Cu) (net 18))
 (segment (start 117.188655 72.992655) (end 115.996047 71.800047) (width 0.25) (layer B.Cu) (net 18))
 (via (at 118.364 73.787) (size 0.8) (drill 0.4) (layers F.Cu B.Cu) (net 18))
 (segment (start 117.188655 72.992655) (end 117.569655 72.992655) (width 0.25) (layer B.Cu) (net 18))
 (segment (start 117.569655 72.992655) (end 118.364 73.787) (width 0.25) (layer B.Cu) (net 18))
 (segment (start 122.936002 73.787) (end 124.650501 72.072501) (width 0.25) (layer F.Cu) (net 18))
 (segment (start 118.364 73.787) (end 122.936002 73.787) (width 0.25) (layer F.Cu) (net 18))
 (segment (start 115.375 71.51) (end 115.375 70.385) (width 0.25) (layer F.Cu) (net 19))
 (segment (start 116.255 72.39) (end 115.375 71.51) (width 0.25) (layer F.Cu) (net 19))
 (segment (start 124.650501 69.532501) (end 121.793002 72.39) (width 0.25) (layer F.Cu) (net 19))
 (segment (start 121.793002 72.39) (end 116.255 72.39) (width 0.25) (layer F.Cu) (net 19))
 (segment (start 116.08606 63.61894) (end 114.395 65.31) (width 0.25) (layer F.Cu) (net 20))
 (segment (start 110.611802 61.727198) (end 111.231163 61.107837) (width 0.25) (layer F.Cu) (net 20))
 (segment (start 114.769011 61.107837) (end 114.949677 61.288503) (width 0.25) (layer F.Cu) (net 20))
 (segment (start 111.231163 61.107837) (end 114.769011 61.107837) (width 0.25) (layer F.Cu) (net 20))
 (segment (start 114.949677 61.288503) (end 115.103672 61.288503) (width 0.25) (layer F.Cu) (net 20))
 (segment (start 114.395 65.31) (end 113.825 65.31) (width 0.25) (layer F.Cu) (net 20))
 (segment (start 116.08606 62.270891) (end 116.08606 63.61894) (width 0.25) (layer F.Cu) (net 20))
 (segment (start 109.410501 64.452501) (end 110.611802 63.2512) (width 0.25) (layer F.Cu) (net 20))
 (segment (start 113.825 65.31) (end 112.7 65.31) (width 0.25) (layer F.Cu) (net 20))
 (segment (start 115.103672 61.288503) (end 116.08606 62.270891) (width 0.25) (layer F.Cu) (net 20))
 (segment (start 110.611802 63.2512) (end 110.611802 61.727198) (width 0.25) (layer F.Cu) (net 20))
 (segment (start 109.410501 66.774499) (end 109.410501 66.992501) (width 0.25) (layer F.Cu) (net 21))
 (segment (start 111.575 64.61) (end 109.410501 66.774499) (width 0.25) (layer F.Cu) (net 21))
 (segment (start 112.7 64.61) (end 111.575 64.61) (width 0.25) (layer F.Cu) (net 21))
 (segment (start 114.174279 64.259279) (end 114.174279 64.380351) (width 0.25) (layer F.Cu) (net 22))
 (segment (start 114.174279 64.768723) (end 114.174279 64.380351) (width 0.25) (layer B.Cu) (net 22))
 (segment (start 112.7 63.91) (end 113.825 63.91) (width 0.25) (layer F.Cu) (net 22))
 (via (at 114.174279 64.380351) (size 0.8) (drill 0.4) (layers F.Cu B.Cu) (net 22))
 (segment (start 109.410501 69.532501) (end 114.174279 64.768723) (width 0.25) (layer B.Cu) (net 22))
 (segment (start 113.825 63.91) (end 114.174279 64.259279) (width 0.25) (layer F.Cu) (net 22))
 (segment (start 114.235964 65.39167) (end 114.899281 64.728353) (width 0.25) (layer B.Cu) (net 23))
 (segment (start 114.235964 65.850036) (end 114.235964 65.39167) (width 0.25) (layer B.Cu) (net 23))
 (segment (start 109.410501 72.072501) (end 109.410501 71.310427) (width 0.25) (layer B.Cu) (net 23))
 (segment (start 110.611802 70.109126) (end 110.611802 69.474198) (width 0.25) (layer B.Cu) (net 23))
 (segment (start 110.611802 69.474198) (end 114.235964 65.850036) (width 0.25) (layer B.Cu) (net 23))
 (segment (start 109.410501 71.310427) (end 110.611802 70.109126) (width 0.25) (layer B.Cu) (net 23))
 (segment (start 114.899281 63.789221) (end 114.573576 63.463516) (width 0.25) (layer B.Cu) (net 23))
 (via (at 114.573576 63.463516) (size 0.8) (drill 0.4) (layers F.Cu B.Cu) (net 23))
 (segment (start 114.899281 64.728353) (end 114.899281 63.789221) (width 0.25) (layer B.Cu) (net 23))
 (segment (start 112.7 63.21) (end 114.32006 63.21) (width 0.25) (layer F.Cu) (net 23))
 (segment (start 114.32006 63.21) (end 114.573576 63.463516) (width 0.25) (layer F.Cu) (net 23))
 (via (at 115.36105 62.833993) (size 0.8) (drill 0.4) (layers F.Cu B.Cu) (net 24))
 (segment (start 115.265571 62.738514) (end 115.36105 62.833993) (width 0.25) (layer F.Cu) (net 24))
 (segment (start 114.207551 62.51) (end 114.436065 62.738514) (width 0.25) (layer F.Cu) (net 24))
 (segment (start 112.7 62.51) (end 114.207551 62.51) (width 0.25) (layer F.Cu) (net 24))
 (segment (start 114.436065 62.738514) (end 115.265571 62.738514) (width 0.25) (layer F.Cu) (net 24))
 (segment (start 114.685975 65.908025) (end 115.36105 65.23295) (width 0.25) (layer B.Cu) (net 24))
 (segment (start 114.685975 66.289025) (end 114.685975 65.908025) (width 0.25) (layer B.Cu) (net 24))
 (segment (start 111.061813 69.913187) (end 114.685975 66.289025) (width 0.25) (layer B.Cu) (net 24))
 (segment (start 115.36105 65.23295) (end 115.36105 63.399678) (width 0.25) (layer B.Cu) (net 24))
 (segment (start 115.36105 63.399678) (end 115.36105 62.833993) (width 0.25) (layer B.Cu) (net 24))
 (segment (start 110.617 73.914) (end 110.617 72.654324) (width 0.25) (layer B.Cu) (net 24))
 (segment (start 109.410501 74.612501) (end 109.918499 74.612501) (width 0.25) (layer B.Cu) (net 24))
 (segment (start 109.918499 74.612501) (end 110.617 73.914) (width 0.25) (layer B.Cu) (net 24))
 (segment (start 110.611802 72.649126) (end 110.611802 70.745536) (width 0.25) (layer B.Cu) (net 24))
 (segment (start 110.617 72.654324) (end 110.611802 72.649126) (width 0.25) (layer B.Cu) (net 24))
 (segment (start 110.611802 70.745536) (end 111.061813 70.295526) (width 0.25) (layer B.Cu) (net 24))
 (segment (start 111.061813 70.295526) (end 111.061813 69.913187) (width 0.25) (layer B.Cu) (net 24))
 (via (at 114.784101 62.013504) (size 0.8) (drill 0.4) (layers F.Cu B.Cu) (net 25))
 (segment (start 112.7 61.81) (end 114.580597 61.81) (width 0.25) (layer F.Cu) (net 25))
 (segment (start 114.580597 61.81) (end 114.784101 62.013504) (width 0.25) (layer F.Cu) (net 25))
 (segment (start 109.410501 77.152501) (end 111.067011 75.495991) (width 0.25) (layer B.Cu) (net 25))
 (segment (start 113.193999 68.799748) (end 113.193999 68.431576) (width 0.25) (layer B.Cu) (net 25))
 (segment (start 116.135989 65.489586) (end 116.135989 62.553451) (width 0.25) (layer B.Cu) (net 25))
 (segment (start 115.349786 62.013504) (end 114.784101 62.013504) (width 0.25) (layer B.Cu) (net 25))
 (segment (start 116.135989 62.553451) (end 115.596042 62.013504) (width 0.25) (layer B.Cu) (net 25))
 (segment (start 115.596042 62.013504) (end 115.349786 62.013504) (width 0.25) (layer B.Cu) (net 25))
 (segment (start 111.067011 70.926736) (end 113.193999 68.799748) (width 0.25) (layer B.Cu) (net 25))
 (segment (start 113.193999 68.431576) (end 116.135989 65.489586) (width 0.25) (layer B.Cu) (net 25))
 (segment (start 111.067011 75.495991) (end 111.067011 70.926736) (width 0.25) (layer B.Cu) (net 25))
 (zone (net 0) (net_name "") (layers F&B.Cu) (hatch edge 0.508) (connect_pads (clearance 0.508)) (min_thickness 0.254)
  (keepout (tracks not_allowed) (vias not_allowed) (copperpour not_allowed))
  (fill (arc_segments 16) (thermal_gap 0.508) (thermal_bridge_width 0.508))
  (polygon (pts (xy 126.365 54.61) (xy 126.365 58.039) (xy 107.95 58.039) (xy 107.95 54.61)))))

